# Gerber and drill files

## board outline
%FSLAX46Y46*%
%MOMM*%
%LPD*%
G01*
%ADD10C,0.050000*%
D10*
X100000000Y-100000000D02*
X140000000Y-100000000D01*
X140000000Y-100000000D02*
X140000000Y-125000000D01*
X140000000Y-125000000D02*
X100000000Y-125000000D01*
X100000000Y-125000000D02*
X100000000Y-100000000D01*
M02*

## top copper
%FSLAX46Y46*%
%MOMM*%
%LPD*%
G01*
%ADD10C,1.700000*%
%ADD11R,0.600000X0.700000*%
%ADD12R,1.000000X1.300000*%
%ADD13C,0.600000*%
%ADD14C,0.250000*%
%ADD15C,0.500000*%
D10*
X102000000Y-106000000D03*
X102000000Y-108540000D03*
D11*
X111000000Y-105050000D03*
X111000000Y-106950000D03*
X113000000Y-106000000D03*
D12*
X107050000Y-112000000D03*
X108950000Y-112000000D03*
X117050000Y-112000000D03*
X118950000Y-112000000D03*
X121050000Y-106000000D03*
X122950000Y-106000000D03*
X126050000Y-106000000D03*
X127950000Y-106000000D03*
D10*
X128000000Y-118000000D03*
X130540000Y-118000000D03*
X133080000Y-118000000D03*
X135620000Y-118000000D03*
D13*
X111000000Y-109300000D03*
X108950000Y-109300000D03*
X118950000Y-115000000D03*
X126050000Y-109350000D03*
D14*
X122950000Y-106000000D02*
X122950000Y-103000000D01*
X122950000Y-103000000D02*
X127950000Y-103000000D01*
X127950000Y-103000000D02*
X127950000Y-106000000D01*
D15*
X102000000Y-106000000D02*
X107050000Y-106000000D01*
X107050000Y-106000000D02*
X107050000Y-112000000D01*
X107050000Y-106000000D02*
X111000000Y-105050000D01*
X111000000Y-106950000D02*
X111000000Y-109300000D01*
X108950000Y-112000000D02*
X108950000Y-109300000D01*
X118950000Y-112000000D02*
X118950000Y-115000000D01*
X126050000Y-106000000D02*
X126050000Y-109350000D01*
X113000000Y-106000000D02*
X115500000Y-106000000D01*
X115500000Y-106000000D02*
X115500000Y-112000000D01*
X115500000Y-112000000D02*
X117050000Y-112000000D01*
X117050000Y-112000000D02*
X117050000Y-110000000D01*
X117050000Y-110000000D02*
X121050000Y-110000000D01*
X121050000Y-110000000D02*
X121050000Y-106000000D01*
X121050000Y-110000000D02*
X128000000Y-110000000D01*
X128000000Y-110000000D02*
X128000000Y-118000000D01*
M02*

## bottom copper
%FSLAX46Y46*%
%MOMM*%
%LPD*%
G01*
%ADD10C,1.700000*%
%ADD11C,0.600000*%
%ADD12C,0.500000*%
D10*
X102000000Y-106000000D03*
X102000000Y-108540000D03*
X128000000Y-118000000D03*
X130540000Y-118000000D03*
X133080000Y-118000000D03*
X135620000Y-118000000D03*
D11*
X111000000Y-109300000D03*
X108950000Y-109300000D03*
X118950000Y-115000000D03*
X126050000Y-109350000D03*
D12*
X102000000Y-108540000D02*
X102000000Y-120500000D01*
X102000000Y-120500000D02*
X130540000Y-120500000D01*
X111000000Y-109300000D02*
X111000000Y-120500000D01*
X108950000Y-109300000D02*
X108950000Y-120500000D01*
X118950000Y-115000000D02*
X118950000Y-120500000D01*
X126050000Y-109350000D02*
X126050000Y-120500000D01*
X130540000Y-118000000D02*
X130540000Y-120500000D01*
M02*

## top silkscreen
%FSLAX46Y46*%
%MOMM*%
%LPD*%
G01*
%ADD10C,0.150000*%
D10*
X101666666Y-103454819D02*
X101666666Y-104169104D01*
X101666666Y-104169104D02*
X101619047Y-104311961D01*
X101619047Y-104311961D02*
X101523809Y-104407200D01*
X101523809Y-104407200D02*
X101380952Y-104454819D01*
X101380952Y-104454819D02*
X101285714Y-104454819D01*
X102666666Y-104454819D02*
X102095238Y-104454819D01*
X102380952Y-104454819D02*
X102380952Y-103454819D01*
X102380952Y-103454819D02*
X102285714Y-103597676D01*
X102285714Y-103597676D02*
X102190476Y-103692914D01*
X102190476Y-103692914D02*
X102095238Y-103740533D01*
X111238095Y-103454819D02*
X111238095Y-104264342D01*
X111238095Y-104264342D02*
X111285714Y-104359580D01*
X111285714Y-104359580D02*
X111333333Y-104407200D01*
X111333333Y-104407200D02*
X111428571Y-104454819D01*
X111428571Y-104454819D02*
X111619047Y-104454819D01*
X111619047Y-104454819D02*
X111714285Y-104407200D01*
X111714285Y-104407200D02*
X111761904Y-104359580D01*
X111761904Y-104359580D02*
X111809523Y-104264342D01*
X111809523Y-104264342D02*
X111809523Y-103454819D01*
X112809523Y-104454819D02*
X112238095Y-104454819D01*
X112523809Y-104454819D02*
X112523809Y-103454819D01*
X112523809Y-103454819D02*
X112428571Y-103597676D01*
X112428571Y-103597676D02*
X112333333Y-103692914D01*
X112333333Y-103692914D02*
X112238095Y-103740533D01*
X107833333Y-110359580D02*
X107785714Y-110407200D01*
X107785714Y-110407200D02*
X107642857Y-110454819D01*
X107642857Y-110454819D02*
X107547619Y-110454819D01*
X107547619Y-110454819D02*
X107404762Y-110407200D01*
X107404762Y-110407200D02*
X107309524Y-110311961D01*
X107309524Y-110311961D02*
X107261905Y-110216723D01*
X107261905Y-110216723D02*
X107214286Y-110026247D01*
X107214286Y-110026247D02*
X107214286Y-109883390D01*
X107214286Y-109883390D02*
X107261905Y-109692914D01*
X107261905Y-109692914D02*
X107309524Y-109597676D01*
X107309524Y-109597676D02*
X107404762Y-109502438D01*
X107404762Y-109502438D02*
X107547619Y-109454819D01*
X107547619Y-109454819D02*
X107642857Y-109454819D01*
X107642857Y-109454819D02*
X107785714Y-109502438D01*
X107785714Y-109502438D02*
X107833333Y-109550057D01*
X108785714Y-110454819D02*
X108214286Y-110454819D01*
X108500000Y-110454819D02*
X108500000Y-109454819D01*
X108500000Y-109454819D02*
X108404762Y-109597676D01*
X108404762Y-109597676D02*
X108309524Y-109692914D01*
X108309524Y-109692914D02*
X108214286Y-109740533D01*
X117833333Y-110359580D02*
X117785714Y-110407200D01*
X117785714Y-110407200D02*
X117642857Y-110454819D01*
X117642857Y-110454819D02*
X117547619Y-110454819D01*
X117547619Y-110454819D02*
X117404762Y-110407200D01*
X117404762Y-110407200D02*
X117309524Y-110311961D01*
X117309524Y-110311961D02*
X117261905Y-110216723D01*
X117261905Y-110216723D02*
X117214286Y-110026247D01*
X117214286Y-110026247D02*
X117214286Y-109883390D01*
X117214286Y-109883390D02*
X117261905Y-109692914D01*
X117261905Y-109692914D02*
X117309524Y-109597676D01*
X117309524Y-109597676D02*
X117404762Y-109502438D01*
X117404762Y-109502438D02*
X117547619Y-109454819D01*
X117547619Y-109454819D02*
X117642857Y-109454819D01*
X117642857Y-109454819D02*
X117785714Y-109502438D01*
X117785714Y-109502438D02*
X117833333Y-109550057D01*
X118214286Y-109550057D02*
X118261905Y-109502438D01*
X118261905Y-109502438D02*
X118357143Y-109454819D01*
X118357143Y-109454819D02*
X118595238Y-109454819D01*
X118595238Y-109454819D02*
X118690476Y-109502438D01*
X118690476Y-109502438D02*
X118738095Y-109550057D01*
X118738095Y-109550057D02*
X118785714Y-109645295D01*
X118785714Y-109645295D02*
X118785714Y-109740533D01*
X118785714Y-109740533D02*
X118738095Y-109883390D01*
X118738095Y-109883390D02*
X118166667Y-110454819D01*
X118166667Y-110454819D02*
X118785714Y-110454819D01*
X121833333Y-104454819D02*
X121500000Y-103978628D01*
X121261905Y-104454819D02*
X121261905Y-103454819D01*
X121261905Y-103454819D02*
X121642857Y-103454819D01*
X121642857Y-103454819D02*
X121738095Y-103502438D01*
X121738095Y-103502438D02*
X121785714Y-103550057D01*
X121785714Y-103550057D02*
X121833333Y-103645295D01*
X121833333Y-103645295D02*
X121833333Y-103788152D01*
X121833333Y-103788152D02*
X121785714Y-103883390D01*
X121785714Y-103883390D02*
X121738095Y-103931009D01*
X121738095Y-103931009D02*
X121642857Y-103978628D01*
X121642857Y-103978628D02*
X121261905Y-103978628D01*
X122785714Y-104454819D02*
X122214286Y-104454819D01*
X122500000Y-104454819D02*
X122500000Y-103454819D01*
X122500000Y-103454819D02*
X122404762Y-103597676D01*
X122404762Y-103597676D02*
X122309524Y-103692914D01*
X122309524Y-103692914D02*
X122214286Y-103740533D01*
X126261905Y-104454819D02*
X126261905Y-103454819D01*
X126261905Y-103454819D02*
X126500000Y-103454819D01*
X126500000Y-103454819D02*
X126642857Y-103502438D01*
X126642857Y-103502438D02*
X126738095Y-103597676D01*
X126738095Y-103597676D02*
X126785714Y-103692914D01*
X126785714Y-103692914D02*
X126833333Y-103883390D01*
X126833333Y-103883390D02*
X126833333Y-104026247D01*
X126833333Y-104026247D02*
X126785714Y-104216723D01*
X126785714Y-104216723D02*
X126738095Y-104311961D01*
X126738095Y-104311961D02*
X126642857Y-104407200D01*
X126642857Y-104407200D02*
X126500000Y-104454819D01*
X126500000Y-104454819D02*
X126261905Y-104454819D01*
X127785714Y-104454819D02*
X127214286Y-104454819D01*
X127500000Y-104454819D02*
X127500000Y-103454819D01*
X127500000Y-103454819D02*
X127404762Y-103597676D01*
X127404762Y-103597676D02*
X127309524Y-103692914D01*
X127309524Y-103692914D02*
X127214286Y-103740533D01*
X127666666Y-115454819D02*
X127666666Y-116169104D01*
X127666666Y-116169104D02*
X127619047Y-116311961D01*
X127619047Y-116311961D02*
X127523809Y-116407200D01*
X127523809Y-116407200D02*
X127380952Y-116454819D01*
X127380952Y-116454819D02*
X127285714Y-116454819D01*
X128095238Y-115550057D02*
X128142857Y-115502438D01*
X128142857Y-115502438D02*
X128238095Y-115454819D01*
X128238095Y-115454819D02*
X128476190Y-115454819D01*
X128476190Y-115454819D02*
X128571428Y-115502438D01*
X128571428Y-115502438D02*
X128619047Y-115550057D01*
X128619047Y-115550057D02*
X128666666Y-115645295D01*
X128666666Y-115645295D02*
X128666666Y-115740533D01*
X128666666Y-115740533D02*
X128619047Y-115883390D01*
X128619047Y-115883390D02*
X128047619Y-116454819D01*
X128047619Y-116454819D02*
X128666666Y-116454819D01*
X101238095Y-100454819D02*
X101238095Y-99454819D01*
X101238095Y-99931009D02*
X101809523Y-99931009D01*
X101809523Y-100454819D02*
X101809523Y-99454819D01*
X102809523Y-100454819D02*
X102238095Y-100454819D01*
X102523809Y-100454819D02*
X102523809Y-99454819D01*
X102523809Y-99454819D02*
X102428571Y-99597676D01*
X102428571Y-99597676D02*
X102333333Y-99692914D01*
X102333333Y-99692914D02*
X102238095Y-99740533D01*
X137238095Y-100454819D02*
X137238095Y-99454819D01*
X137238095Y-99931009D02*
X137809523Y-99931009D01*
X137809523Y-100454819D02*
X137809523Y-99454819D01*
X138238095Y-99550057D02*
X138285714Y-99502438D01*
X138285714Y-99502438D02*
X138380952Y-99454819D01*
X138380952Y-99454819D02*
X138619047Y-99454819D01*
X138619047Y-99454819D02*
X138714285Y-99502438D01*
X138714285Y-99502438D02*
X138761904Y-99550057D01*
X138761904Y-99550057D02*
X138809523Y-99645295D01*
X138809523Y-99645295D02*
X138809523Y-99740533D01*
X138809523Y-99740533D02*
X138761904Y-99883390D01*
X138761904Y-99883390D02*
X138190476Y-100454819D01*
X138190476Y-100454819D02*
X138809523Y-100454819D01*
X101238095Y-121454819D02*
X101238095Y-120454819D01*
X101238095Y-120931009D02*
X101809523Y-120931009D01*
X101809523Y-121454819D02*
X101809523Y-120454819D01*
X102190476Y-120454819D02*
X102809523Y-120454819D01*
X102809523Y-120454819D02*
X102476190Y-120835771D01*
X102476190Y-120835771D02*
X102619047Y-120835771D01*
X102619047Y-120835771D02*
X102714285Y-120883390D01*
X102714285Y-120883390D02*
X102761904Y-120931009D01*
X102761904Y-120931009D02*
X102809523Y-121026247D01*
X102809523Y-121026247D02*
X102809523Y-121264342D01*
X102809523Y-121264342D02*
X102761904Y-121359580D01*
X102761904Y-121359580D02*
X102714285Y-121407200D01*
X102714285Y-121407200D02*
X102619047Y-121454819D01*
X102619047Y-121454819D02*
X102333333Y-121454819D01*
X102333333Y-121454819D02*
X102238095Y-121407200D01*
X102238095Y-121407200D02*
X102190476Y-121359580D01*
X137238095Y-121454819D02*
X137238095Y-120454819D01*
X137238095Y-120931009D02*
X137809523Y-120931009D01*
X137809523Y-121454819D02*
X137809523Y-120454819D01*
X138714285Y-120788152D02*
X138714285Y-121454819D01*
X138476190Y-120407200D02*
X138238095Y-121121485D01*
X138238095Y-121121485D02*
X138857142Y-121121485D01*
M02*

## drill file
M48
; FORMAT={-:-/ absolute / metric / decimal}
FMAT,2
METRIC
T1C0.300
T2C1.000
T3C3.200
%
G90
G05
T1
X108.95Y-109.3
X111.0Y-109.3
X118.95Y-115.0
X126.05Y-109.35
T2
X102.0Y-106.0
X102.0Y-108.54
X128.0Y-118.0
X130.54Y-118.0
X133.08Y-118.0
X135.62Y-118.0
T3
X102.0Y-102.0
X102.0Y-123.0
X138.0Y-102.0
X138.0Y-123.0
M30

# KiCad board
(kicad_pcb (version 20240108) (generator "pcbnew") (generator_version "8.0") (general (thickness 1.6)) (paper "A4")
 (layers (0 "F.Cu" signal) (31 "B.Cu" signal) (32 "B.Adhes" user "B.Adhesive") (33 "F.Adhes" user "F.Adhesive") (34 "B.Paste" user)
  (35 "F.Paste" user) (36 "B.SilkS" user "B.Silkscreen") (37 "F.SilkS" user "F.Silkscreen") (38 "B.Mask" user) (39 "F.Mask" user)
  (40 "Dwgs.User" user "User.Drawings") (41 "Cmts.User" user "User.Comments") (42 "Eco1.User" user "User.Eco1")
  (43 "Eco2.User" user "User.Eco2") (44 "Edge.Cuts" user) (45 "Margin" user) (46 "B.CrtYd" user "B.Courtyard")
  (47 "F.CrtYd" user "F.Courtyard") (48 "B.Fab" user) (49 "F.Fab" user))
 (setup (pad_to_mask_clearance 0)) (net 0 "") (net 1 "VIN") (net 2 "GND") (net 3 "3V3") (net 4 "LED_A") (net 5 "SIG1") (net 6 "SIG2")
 (gr_line (start 100 100) (end 140 100) (stroke (width 0.05) (type default)) (layer "Edge.Cuts"))
 (gr_line (start 140 100) (end 140 125) (stroke (width 0.05) (type default)) (layer "Edge.Cuts"))
 (gr_line (start 140 125) (end 100 125) (stroke (width 0.05) (type default)) (layer "Edge.Cuts"))
 (gr_line (start 100 125) (end 100 100) (stroke (width 0.05) (type default)) (layer "Edge.Cuts"))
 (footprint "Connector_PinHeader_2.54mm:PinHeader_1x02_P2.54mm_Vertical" (layer "F.Cu") (at 102 106)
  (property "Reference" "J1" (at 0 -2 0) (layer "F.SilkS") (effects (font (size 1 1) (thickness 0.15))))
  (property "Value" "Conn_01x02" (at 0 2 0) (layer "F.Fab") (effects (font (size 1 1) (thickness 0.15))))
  (pad "1" thru_hole circle (at 0 0) (size 1.7 1.7) (drill 1) (layers "*.Cu" "*.Mask") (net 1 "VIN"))
  (pad "2" thru_hole circle (at 0 2.54) (size 1.7 1.7) (drill 1) (layers "*.Cu" "*.Mask") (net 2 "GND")))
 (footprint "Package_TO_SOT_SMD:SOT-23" (layer "F.Cu") (at 112 106)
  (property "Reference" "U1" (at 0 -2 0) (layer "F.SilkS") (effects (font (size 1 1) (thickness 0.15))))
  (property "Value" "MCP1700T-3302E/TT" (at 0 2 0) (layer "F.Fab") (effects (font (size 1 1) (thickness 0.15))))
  (pad "1" smd rect (at -1 -0.95) (size 0.6 0.7) (layers "F.Cu" "F.Paste" "F.Mask") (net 1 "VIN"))
  (pad "2" smd rect (at -1 0.95) (size 0.6 0.7) (layers "F.Cu" "F.Paste" "F.Mask") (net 2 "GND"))
  (pad "3" smd rect (at 1 0) (size 0.6 0.7) (layers "F.Cu" "F.Paste" "F.Mask") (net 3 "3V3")))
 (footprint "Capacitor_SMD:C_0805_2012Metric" (layer "F.Cu") (at 108 112)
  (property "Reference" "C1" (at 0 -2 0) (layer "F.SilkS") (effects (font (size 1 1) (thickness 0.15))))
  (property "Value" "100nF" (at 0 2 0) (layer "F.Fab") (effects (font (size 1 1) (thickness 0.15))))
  (pad "1" smd rect (at -0.95 0) (size 1 1.3) (layers "F.Cu" "F.Paste" "F.Mask") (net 1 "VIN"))
  (pad "2" smd rect (at 0.95 0) (size 1 1.3) (layers "F.Cu" "F.Paste" "F.Mask") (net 2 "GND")))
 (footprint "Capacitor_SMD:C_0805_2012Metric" (layer "F.Cu") (at 118 112)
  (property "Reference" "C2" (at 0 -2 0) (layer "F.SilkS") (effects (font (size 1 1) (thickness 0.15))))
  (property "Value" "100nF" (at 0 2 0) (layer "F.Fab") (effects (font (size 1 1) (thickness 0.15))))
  (pad "1" smd rect (at -0.95 0) (size 1 1.3) (layers "F.Cu" "F.Paste" "F.Mask") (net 3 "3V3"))
  (pad "2" smd rect (at 0.95 0) (size 1 1.3) (layers "F.Cu" "F.Paste" "F.Mask") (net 2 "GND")))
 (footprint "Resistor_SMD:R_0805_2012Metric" (layer "F.Cu") (at 122 106)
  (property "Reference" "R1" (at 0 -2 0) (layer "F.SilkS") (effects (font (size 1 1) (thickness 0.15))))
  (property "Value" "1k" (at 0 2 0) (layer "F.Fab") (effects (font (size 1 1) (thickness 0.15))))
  (pad "1" smd rect (at -0.95 0) (size 1 1.3) (layers "F.Cu" "F.Paste" "F.Mask") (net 3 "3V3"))
  (pad "2" smd rect (at 0.95 0) (size 1 1.3) (layers "F.Cu" "F.Paste" "F.Mask") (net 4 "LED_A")))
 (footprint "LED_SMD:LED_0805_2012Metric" (layer "F.Cu") (at 127 106)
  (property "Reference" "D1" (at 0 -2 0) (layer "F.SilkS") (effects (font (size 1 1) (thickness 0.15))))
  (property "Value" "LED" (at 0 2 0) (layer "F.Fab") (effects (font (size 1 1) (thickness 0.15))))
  (pad "1" smd rect (at -0.95 0) (size 1 1.3) (layers "F.Cu" "F.Paste" "F.Mask") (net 2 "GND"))
  (pad "2" smd rect (at 0.95 0) (size 1 1.3) (layers "F.Cu" "F.Paste" "F.Mask") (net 4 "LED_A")))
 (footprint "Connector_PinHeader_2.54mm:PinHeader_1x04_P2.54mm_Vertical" (layer "F.Cu") (at 128 118)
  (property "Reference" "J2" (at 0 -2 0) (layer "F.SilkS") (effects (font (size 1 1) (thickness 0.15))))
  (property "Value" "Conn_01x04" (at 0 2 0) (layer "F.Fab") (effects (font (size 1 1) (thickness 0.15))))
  (pad "1" thru_hole circle (at 0 0) (size 1.7 1.7) (drill 1) (layers "*.Cu" "*.Mask") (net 3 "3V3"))
  (pad "2" thru_hole circle (at 2.54 0) (size 1.7 1.7) (drill 1) (layers "*.Cu" "*.Mask") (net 2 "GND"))
  (pad "3" thru_hole circle (at 5.08 0) (size 1.7 1.7) (drill 1) (layers "*.Cu" "*.Mask") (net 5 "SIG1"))
  (pad "4" thru_hole circle (at 7.62 0) (size 1.7 1.7) (drill 1) (layers "*.Cu" "*.Mask") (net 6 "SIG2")))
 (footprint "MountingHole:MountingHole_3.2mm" (layer "F.Cu") (at 102 102)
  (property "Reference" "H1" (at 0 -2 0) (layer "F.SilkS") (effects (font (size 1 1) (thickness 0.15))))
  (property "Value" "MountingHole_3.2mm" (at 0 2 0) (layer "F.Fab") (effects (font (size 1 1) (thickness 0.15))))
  (pad "1" np_thru_hole circle (at 0 0) (size 3.2 3.2) (drill 3.2) (layers "*.Cu" "*.Mask")))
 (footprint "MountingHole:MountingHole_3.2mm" (layer "F.Cu") (at 138 102)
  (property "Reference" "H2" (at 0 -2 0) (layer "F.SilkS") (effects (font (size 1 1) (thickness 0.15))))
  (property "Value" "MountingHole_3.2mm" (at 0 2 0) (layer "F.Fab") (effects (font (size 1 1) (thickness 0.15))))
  (pad "1" np_thru_hole circle (at 0 0) (size 3.2 3.2) (drill 3.2) (layers "*.Cu" "*.Mask")))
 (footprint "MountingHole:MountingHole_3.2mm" (layer "F.Cu") (at 102 123)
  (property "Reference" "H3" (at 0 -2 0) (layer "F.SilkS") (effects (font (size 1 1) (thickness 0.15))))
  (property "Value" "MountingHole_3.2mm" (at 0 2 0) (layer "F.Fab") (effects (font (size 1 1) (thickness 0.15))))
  (pad "1" np_thru_hole circle (at 0 0) (size 3.2 3.2) (drill 3.2) (layers "*.Cu" "*.Mask")))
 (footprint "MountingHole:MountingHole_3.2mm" (layer "F.Cu") (at 138 123)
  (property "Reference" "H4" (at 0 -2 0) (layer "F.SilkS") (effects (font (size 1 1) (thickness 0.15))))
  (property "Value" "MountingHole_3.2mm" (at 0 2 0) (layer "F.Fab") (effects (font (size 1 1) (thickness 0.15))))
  (pad "1" np_thru_hole circle (at 0 0) (size 3.2 3.2) (drill 3.2) (layers "*.Cu" "*.Mask")))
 (segment (start 122.95 106) (end 122.95 103) (width 0.25) (layer "F.Cu") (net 4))
 (segment (start 122.95 103) (end 127.95 103) (width 0.25) (layer "F.Cu") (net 4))
 (segment (start 127.95 103) (end 127.95 106) (width 0.25) (layer "F.Cu") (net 4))
 (segment (start 102 106) (end 107.05 106) (width 0.5) (layer "F.Cu") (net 1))
 (segment (start 107.05 106) (end 107.05 112) (width 0.5) (layer "F.Cu") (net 1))
 (segment (start 107.05 106) (end 111 105.05) (width 0.5) (layer "F.Cu") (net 1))
 (segment (start 111 106.95) (end 111 109.3) (width 0.5) (layer "F.Cu") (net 2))
 (segment (start 108.95 112) (end 108.95 109.3) (width 0.5) (layer "F.Cu") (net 2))
 (segment (start 118.95 112) (end 118.95 115) (width 0.5) (layer "F.Cu") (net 2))
 (segment (start 126.05 106) (end 126.05 109.35) (width 0.5) (layer "F.Cu") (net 2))
 (segment (start 113 106) (end 115.5 106) (width 0.5) (layer "F.Cu") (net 3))
 (segment (start 115.5 106) (end 115.5 112) (width 0.5) (layer "F.Cu") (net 3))
 (segment (start 115.5 112) (end 117.05 112) (width 0.5) (layer "F.Cu") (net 3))
 (segment (start 117.05 112) (end 117.05 110) (width 0.5) (layer "F.Cu") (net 3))
 (segment (start 117.05 110) (end 121.05 110) (width 0.5) (layer "F.Cu") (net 3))
 (segment (start 121.05 110) (end 121.05 106) (width 0.5) (layer "F.Cu") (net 3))
 (segment (start 121.05 110) (end 128 110) (width 0.5) (layer "F.Cu") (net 3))
 (segment (start 128 110) (end 128 118) (width 0.5) (layer "F.Cu") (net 3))
 (segment (start 102 108.54) (end 102 120.5) (width 0.5) (layer "B.Cu") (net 2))
 (segment (start 102 120.5) (end 130.54 120.5) (width 0.5) (layer "B.Cu") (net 2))
 (segment (start 111 109.3) (end 111 120.5) (width 0.5) (layer "B.Cu") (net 2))
 (segment (start 108.95 109.3) (end 108.95 120.5) (width 0.5) (layer "B.Cu") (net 2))
 (segment (start 118.95 115) (end 118.95 120.5) (width 0.5) (layer "B.Cu") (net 2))
 (segment (start 126.05 109.35) (end 126.05 120.5) (width 0.5) (layer "B.Cu") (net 2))
 (segment (start 130.54 118) (end 130.54 120.5) (width 0.5) (layer "B.Cu") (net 2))
 (via (at 111 109.3) (size 0.6) (drill 0.3) (layers "F.Cu" "B.Cu") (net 2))
 (via (at 108.95 109.3) (size 0.6) (drill 0.3) (layers "F.Cu" "B.Cu") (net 2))
 (via (at 118.95 115) (size 0.6) (drill 0.3) (layers "F.Cu" "B.Cu") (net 2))
 (via (at 126.05 109.35) (size 0.6) (drill 0.3) (layers "F.Cu" "B.Cu") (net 2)))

